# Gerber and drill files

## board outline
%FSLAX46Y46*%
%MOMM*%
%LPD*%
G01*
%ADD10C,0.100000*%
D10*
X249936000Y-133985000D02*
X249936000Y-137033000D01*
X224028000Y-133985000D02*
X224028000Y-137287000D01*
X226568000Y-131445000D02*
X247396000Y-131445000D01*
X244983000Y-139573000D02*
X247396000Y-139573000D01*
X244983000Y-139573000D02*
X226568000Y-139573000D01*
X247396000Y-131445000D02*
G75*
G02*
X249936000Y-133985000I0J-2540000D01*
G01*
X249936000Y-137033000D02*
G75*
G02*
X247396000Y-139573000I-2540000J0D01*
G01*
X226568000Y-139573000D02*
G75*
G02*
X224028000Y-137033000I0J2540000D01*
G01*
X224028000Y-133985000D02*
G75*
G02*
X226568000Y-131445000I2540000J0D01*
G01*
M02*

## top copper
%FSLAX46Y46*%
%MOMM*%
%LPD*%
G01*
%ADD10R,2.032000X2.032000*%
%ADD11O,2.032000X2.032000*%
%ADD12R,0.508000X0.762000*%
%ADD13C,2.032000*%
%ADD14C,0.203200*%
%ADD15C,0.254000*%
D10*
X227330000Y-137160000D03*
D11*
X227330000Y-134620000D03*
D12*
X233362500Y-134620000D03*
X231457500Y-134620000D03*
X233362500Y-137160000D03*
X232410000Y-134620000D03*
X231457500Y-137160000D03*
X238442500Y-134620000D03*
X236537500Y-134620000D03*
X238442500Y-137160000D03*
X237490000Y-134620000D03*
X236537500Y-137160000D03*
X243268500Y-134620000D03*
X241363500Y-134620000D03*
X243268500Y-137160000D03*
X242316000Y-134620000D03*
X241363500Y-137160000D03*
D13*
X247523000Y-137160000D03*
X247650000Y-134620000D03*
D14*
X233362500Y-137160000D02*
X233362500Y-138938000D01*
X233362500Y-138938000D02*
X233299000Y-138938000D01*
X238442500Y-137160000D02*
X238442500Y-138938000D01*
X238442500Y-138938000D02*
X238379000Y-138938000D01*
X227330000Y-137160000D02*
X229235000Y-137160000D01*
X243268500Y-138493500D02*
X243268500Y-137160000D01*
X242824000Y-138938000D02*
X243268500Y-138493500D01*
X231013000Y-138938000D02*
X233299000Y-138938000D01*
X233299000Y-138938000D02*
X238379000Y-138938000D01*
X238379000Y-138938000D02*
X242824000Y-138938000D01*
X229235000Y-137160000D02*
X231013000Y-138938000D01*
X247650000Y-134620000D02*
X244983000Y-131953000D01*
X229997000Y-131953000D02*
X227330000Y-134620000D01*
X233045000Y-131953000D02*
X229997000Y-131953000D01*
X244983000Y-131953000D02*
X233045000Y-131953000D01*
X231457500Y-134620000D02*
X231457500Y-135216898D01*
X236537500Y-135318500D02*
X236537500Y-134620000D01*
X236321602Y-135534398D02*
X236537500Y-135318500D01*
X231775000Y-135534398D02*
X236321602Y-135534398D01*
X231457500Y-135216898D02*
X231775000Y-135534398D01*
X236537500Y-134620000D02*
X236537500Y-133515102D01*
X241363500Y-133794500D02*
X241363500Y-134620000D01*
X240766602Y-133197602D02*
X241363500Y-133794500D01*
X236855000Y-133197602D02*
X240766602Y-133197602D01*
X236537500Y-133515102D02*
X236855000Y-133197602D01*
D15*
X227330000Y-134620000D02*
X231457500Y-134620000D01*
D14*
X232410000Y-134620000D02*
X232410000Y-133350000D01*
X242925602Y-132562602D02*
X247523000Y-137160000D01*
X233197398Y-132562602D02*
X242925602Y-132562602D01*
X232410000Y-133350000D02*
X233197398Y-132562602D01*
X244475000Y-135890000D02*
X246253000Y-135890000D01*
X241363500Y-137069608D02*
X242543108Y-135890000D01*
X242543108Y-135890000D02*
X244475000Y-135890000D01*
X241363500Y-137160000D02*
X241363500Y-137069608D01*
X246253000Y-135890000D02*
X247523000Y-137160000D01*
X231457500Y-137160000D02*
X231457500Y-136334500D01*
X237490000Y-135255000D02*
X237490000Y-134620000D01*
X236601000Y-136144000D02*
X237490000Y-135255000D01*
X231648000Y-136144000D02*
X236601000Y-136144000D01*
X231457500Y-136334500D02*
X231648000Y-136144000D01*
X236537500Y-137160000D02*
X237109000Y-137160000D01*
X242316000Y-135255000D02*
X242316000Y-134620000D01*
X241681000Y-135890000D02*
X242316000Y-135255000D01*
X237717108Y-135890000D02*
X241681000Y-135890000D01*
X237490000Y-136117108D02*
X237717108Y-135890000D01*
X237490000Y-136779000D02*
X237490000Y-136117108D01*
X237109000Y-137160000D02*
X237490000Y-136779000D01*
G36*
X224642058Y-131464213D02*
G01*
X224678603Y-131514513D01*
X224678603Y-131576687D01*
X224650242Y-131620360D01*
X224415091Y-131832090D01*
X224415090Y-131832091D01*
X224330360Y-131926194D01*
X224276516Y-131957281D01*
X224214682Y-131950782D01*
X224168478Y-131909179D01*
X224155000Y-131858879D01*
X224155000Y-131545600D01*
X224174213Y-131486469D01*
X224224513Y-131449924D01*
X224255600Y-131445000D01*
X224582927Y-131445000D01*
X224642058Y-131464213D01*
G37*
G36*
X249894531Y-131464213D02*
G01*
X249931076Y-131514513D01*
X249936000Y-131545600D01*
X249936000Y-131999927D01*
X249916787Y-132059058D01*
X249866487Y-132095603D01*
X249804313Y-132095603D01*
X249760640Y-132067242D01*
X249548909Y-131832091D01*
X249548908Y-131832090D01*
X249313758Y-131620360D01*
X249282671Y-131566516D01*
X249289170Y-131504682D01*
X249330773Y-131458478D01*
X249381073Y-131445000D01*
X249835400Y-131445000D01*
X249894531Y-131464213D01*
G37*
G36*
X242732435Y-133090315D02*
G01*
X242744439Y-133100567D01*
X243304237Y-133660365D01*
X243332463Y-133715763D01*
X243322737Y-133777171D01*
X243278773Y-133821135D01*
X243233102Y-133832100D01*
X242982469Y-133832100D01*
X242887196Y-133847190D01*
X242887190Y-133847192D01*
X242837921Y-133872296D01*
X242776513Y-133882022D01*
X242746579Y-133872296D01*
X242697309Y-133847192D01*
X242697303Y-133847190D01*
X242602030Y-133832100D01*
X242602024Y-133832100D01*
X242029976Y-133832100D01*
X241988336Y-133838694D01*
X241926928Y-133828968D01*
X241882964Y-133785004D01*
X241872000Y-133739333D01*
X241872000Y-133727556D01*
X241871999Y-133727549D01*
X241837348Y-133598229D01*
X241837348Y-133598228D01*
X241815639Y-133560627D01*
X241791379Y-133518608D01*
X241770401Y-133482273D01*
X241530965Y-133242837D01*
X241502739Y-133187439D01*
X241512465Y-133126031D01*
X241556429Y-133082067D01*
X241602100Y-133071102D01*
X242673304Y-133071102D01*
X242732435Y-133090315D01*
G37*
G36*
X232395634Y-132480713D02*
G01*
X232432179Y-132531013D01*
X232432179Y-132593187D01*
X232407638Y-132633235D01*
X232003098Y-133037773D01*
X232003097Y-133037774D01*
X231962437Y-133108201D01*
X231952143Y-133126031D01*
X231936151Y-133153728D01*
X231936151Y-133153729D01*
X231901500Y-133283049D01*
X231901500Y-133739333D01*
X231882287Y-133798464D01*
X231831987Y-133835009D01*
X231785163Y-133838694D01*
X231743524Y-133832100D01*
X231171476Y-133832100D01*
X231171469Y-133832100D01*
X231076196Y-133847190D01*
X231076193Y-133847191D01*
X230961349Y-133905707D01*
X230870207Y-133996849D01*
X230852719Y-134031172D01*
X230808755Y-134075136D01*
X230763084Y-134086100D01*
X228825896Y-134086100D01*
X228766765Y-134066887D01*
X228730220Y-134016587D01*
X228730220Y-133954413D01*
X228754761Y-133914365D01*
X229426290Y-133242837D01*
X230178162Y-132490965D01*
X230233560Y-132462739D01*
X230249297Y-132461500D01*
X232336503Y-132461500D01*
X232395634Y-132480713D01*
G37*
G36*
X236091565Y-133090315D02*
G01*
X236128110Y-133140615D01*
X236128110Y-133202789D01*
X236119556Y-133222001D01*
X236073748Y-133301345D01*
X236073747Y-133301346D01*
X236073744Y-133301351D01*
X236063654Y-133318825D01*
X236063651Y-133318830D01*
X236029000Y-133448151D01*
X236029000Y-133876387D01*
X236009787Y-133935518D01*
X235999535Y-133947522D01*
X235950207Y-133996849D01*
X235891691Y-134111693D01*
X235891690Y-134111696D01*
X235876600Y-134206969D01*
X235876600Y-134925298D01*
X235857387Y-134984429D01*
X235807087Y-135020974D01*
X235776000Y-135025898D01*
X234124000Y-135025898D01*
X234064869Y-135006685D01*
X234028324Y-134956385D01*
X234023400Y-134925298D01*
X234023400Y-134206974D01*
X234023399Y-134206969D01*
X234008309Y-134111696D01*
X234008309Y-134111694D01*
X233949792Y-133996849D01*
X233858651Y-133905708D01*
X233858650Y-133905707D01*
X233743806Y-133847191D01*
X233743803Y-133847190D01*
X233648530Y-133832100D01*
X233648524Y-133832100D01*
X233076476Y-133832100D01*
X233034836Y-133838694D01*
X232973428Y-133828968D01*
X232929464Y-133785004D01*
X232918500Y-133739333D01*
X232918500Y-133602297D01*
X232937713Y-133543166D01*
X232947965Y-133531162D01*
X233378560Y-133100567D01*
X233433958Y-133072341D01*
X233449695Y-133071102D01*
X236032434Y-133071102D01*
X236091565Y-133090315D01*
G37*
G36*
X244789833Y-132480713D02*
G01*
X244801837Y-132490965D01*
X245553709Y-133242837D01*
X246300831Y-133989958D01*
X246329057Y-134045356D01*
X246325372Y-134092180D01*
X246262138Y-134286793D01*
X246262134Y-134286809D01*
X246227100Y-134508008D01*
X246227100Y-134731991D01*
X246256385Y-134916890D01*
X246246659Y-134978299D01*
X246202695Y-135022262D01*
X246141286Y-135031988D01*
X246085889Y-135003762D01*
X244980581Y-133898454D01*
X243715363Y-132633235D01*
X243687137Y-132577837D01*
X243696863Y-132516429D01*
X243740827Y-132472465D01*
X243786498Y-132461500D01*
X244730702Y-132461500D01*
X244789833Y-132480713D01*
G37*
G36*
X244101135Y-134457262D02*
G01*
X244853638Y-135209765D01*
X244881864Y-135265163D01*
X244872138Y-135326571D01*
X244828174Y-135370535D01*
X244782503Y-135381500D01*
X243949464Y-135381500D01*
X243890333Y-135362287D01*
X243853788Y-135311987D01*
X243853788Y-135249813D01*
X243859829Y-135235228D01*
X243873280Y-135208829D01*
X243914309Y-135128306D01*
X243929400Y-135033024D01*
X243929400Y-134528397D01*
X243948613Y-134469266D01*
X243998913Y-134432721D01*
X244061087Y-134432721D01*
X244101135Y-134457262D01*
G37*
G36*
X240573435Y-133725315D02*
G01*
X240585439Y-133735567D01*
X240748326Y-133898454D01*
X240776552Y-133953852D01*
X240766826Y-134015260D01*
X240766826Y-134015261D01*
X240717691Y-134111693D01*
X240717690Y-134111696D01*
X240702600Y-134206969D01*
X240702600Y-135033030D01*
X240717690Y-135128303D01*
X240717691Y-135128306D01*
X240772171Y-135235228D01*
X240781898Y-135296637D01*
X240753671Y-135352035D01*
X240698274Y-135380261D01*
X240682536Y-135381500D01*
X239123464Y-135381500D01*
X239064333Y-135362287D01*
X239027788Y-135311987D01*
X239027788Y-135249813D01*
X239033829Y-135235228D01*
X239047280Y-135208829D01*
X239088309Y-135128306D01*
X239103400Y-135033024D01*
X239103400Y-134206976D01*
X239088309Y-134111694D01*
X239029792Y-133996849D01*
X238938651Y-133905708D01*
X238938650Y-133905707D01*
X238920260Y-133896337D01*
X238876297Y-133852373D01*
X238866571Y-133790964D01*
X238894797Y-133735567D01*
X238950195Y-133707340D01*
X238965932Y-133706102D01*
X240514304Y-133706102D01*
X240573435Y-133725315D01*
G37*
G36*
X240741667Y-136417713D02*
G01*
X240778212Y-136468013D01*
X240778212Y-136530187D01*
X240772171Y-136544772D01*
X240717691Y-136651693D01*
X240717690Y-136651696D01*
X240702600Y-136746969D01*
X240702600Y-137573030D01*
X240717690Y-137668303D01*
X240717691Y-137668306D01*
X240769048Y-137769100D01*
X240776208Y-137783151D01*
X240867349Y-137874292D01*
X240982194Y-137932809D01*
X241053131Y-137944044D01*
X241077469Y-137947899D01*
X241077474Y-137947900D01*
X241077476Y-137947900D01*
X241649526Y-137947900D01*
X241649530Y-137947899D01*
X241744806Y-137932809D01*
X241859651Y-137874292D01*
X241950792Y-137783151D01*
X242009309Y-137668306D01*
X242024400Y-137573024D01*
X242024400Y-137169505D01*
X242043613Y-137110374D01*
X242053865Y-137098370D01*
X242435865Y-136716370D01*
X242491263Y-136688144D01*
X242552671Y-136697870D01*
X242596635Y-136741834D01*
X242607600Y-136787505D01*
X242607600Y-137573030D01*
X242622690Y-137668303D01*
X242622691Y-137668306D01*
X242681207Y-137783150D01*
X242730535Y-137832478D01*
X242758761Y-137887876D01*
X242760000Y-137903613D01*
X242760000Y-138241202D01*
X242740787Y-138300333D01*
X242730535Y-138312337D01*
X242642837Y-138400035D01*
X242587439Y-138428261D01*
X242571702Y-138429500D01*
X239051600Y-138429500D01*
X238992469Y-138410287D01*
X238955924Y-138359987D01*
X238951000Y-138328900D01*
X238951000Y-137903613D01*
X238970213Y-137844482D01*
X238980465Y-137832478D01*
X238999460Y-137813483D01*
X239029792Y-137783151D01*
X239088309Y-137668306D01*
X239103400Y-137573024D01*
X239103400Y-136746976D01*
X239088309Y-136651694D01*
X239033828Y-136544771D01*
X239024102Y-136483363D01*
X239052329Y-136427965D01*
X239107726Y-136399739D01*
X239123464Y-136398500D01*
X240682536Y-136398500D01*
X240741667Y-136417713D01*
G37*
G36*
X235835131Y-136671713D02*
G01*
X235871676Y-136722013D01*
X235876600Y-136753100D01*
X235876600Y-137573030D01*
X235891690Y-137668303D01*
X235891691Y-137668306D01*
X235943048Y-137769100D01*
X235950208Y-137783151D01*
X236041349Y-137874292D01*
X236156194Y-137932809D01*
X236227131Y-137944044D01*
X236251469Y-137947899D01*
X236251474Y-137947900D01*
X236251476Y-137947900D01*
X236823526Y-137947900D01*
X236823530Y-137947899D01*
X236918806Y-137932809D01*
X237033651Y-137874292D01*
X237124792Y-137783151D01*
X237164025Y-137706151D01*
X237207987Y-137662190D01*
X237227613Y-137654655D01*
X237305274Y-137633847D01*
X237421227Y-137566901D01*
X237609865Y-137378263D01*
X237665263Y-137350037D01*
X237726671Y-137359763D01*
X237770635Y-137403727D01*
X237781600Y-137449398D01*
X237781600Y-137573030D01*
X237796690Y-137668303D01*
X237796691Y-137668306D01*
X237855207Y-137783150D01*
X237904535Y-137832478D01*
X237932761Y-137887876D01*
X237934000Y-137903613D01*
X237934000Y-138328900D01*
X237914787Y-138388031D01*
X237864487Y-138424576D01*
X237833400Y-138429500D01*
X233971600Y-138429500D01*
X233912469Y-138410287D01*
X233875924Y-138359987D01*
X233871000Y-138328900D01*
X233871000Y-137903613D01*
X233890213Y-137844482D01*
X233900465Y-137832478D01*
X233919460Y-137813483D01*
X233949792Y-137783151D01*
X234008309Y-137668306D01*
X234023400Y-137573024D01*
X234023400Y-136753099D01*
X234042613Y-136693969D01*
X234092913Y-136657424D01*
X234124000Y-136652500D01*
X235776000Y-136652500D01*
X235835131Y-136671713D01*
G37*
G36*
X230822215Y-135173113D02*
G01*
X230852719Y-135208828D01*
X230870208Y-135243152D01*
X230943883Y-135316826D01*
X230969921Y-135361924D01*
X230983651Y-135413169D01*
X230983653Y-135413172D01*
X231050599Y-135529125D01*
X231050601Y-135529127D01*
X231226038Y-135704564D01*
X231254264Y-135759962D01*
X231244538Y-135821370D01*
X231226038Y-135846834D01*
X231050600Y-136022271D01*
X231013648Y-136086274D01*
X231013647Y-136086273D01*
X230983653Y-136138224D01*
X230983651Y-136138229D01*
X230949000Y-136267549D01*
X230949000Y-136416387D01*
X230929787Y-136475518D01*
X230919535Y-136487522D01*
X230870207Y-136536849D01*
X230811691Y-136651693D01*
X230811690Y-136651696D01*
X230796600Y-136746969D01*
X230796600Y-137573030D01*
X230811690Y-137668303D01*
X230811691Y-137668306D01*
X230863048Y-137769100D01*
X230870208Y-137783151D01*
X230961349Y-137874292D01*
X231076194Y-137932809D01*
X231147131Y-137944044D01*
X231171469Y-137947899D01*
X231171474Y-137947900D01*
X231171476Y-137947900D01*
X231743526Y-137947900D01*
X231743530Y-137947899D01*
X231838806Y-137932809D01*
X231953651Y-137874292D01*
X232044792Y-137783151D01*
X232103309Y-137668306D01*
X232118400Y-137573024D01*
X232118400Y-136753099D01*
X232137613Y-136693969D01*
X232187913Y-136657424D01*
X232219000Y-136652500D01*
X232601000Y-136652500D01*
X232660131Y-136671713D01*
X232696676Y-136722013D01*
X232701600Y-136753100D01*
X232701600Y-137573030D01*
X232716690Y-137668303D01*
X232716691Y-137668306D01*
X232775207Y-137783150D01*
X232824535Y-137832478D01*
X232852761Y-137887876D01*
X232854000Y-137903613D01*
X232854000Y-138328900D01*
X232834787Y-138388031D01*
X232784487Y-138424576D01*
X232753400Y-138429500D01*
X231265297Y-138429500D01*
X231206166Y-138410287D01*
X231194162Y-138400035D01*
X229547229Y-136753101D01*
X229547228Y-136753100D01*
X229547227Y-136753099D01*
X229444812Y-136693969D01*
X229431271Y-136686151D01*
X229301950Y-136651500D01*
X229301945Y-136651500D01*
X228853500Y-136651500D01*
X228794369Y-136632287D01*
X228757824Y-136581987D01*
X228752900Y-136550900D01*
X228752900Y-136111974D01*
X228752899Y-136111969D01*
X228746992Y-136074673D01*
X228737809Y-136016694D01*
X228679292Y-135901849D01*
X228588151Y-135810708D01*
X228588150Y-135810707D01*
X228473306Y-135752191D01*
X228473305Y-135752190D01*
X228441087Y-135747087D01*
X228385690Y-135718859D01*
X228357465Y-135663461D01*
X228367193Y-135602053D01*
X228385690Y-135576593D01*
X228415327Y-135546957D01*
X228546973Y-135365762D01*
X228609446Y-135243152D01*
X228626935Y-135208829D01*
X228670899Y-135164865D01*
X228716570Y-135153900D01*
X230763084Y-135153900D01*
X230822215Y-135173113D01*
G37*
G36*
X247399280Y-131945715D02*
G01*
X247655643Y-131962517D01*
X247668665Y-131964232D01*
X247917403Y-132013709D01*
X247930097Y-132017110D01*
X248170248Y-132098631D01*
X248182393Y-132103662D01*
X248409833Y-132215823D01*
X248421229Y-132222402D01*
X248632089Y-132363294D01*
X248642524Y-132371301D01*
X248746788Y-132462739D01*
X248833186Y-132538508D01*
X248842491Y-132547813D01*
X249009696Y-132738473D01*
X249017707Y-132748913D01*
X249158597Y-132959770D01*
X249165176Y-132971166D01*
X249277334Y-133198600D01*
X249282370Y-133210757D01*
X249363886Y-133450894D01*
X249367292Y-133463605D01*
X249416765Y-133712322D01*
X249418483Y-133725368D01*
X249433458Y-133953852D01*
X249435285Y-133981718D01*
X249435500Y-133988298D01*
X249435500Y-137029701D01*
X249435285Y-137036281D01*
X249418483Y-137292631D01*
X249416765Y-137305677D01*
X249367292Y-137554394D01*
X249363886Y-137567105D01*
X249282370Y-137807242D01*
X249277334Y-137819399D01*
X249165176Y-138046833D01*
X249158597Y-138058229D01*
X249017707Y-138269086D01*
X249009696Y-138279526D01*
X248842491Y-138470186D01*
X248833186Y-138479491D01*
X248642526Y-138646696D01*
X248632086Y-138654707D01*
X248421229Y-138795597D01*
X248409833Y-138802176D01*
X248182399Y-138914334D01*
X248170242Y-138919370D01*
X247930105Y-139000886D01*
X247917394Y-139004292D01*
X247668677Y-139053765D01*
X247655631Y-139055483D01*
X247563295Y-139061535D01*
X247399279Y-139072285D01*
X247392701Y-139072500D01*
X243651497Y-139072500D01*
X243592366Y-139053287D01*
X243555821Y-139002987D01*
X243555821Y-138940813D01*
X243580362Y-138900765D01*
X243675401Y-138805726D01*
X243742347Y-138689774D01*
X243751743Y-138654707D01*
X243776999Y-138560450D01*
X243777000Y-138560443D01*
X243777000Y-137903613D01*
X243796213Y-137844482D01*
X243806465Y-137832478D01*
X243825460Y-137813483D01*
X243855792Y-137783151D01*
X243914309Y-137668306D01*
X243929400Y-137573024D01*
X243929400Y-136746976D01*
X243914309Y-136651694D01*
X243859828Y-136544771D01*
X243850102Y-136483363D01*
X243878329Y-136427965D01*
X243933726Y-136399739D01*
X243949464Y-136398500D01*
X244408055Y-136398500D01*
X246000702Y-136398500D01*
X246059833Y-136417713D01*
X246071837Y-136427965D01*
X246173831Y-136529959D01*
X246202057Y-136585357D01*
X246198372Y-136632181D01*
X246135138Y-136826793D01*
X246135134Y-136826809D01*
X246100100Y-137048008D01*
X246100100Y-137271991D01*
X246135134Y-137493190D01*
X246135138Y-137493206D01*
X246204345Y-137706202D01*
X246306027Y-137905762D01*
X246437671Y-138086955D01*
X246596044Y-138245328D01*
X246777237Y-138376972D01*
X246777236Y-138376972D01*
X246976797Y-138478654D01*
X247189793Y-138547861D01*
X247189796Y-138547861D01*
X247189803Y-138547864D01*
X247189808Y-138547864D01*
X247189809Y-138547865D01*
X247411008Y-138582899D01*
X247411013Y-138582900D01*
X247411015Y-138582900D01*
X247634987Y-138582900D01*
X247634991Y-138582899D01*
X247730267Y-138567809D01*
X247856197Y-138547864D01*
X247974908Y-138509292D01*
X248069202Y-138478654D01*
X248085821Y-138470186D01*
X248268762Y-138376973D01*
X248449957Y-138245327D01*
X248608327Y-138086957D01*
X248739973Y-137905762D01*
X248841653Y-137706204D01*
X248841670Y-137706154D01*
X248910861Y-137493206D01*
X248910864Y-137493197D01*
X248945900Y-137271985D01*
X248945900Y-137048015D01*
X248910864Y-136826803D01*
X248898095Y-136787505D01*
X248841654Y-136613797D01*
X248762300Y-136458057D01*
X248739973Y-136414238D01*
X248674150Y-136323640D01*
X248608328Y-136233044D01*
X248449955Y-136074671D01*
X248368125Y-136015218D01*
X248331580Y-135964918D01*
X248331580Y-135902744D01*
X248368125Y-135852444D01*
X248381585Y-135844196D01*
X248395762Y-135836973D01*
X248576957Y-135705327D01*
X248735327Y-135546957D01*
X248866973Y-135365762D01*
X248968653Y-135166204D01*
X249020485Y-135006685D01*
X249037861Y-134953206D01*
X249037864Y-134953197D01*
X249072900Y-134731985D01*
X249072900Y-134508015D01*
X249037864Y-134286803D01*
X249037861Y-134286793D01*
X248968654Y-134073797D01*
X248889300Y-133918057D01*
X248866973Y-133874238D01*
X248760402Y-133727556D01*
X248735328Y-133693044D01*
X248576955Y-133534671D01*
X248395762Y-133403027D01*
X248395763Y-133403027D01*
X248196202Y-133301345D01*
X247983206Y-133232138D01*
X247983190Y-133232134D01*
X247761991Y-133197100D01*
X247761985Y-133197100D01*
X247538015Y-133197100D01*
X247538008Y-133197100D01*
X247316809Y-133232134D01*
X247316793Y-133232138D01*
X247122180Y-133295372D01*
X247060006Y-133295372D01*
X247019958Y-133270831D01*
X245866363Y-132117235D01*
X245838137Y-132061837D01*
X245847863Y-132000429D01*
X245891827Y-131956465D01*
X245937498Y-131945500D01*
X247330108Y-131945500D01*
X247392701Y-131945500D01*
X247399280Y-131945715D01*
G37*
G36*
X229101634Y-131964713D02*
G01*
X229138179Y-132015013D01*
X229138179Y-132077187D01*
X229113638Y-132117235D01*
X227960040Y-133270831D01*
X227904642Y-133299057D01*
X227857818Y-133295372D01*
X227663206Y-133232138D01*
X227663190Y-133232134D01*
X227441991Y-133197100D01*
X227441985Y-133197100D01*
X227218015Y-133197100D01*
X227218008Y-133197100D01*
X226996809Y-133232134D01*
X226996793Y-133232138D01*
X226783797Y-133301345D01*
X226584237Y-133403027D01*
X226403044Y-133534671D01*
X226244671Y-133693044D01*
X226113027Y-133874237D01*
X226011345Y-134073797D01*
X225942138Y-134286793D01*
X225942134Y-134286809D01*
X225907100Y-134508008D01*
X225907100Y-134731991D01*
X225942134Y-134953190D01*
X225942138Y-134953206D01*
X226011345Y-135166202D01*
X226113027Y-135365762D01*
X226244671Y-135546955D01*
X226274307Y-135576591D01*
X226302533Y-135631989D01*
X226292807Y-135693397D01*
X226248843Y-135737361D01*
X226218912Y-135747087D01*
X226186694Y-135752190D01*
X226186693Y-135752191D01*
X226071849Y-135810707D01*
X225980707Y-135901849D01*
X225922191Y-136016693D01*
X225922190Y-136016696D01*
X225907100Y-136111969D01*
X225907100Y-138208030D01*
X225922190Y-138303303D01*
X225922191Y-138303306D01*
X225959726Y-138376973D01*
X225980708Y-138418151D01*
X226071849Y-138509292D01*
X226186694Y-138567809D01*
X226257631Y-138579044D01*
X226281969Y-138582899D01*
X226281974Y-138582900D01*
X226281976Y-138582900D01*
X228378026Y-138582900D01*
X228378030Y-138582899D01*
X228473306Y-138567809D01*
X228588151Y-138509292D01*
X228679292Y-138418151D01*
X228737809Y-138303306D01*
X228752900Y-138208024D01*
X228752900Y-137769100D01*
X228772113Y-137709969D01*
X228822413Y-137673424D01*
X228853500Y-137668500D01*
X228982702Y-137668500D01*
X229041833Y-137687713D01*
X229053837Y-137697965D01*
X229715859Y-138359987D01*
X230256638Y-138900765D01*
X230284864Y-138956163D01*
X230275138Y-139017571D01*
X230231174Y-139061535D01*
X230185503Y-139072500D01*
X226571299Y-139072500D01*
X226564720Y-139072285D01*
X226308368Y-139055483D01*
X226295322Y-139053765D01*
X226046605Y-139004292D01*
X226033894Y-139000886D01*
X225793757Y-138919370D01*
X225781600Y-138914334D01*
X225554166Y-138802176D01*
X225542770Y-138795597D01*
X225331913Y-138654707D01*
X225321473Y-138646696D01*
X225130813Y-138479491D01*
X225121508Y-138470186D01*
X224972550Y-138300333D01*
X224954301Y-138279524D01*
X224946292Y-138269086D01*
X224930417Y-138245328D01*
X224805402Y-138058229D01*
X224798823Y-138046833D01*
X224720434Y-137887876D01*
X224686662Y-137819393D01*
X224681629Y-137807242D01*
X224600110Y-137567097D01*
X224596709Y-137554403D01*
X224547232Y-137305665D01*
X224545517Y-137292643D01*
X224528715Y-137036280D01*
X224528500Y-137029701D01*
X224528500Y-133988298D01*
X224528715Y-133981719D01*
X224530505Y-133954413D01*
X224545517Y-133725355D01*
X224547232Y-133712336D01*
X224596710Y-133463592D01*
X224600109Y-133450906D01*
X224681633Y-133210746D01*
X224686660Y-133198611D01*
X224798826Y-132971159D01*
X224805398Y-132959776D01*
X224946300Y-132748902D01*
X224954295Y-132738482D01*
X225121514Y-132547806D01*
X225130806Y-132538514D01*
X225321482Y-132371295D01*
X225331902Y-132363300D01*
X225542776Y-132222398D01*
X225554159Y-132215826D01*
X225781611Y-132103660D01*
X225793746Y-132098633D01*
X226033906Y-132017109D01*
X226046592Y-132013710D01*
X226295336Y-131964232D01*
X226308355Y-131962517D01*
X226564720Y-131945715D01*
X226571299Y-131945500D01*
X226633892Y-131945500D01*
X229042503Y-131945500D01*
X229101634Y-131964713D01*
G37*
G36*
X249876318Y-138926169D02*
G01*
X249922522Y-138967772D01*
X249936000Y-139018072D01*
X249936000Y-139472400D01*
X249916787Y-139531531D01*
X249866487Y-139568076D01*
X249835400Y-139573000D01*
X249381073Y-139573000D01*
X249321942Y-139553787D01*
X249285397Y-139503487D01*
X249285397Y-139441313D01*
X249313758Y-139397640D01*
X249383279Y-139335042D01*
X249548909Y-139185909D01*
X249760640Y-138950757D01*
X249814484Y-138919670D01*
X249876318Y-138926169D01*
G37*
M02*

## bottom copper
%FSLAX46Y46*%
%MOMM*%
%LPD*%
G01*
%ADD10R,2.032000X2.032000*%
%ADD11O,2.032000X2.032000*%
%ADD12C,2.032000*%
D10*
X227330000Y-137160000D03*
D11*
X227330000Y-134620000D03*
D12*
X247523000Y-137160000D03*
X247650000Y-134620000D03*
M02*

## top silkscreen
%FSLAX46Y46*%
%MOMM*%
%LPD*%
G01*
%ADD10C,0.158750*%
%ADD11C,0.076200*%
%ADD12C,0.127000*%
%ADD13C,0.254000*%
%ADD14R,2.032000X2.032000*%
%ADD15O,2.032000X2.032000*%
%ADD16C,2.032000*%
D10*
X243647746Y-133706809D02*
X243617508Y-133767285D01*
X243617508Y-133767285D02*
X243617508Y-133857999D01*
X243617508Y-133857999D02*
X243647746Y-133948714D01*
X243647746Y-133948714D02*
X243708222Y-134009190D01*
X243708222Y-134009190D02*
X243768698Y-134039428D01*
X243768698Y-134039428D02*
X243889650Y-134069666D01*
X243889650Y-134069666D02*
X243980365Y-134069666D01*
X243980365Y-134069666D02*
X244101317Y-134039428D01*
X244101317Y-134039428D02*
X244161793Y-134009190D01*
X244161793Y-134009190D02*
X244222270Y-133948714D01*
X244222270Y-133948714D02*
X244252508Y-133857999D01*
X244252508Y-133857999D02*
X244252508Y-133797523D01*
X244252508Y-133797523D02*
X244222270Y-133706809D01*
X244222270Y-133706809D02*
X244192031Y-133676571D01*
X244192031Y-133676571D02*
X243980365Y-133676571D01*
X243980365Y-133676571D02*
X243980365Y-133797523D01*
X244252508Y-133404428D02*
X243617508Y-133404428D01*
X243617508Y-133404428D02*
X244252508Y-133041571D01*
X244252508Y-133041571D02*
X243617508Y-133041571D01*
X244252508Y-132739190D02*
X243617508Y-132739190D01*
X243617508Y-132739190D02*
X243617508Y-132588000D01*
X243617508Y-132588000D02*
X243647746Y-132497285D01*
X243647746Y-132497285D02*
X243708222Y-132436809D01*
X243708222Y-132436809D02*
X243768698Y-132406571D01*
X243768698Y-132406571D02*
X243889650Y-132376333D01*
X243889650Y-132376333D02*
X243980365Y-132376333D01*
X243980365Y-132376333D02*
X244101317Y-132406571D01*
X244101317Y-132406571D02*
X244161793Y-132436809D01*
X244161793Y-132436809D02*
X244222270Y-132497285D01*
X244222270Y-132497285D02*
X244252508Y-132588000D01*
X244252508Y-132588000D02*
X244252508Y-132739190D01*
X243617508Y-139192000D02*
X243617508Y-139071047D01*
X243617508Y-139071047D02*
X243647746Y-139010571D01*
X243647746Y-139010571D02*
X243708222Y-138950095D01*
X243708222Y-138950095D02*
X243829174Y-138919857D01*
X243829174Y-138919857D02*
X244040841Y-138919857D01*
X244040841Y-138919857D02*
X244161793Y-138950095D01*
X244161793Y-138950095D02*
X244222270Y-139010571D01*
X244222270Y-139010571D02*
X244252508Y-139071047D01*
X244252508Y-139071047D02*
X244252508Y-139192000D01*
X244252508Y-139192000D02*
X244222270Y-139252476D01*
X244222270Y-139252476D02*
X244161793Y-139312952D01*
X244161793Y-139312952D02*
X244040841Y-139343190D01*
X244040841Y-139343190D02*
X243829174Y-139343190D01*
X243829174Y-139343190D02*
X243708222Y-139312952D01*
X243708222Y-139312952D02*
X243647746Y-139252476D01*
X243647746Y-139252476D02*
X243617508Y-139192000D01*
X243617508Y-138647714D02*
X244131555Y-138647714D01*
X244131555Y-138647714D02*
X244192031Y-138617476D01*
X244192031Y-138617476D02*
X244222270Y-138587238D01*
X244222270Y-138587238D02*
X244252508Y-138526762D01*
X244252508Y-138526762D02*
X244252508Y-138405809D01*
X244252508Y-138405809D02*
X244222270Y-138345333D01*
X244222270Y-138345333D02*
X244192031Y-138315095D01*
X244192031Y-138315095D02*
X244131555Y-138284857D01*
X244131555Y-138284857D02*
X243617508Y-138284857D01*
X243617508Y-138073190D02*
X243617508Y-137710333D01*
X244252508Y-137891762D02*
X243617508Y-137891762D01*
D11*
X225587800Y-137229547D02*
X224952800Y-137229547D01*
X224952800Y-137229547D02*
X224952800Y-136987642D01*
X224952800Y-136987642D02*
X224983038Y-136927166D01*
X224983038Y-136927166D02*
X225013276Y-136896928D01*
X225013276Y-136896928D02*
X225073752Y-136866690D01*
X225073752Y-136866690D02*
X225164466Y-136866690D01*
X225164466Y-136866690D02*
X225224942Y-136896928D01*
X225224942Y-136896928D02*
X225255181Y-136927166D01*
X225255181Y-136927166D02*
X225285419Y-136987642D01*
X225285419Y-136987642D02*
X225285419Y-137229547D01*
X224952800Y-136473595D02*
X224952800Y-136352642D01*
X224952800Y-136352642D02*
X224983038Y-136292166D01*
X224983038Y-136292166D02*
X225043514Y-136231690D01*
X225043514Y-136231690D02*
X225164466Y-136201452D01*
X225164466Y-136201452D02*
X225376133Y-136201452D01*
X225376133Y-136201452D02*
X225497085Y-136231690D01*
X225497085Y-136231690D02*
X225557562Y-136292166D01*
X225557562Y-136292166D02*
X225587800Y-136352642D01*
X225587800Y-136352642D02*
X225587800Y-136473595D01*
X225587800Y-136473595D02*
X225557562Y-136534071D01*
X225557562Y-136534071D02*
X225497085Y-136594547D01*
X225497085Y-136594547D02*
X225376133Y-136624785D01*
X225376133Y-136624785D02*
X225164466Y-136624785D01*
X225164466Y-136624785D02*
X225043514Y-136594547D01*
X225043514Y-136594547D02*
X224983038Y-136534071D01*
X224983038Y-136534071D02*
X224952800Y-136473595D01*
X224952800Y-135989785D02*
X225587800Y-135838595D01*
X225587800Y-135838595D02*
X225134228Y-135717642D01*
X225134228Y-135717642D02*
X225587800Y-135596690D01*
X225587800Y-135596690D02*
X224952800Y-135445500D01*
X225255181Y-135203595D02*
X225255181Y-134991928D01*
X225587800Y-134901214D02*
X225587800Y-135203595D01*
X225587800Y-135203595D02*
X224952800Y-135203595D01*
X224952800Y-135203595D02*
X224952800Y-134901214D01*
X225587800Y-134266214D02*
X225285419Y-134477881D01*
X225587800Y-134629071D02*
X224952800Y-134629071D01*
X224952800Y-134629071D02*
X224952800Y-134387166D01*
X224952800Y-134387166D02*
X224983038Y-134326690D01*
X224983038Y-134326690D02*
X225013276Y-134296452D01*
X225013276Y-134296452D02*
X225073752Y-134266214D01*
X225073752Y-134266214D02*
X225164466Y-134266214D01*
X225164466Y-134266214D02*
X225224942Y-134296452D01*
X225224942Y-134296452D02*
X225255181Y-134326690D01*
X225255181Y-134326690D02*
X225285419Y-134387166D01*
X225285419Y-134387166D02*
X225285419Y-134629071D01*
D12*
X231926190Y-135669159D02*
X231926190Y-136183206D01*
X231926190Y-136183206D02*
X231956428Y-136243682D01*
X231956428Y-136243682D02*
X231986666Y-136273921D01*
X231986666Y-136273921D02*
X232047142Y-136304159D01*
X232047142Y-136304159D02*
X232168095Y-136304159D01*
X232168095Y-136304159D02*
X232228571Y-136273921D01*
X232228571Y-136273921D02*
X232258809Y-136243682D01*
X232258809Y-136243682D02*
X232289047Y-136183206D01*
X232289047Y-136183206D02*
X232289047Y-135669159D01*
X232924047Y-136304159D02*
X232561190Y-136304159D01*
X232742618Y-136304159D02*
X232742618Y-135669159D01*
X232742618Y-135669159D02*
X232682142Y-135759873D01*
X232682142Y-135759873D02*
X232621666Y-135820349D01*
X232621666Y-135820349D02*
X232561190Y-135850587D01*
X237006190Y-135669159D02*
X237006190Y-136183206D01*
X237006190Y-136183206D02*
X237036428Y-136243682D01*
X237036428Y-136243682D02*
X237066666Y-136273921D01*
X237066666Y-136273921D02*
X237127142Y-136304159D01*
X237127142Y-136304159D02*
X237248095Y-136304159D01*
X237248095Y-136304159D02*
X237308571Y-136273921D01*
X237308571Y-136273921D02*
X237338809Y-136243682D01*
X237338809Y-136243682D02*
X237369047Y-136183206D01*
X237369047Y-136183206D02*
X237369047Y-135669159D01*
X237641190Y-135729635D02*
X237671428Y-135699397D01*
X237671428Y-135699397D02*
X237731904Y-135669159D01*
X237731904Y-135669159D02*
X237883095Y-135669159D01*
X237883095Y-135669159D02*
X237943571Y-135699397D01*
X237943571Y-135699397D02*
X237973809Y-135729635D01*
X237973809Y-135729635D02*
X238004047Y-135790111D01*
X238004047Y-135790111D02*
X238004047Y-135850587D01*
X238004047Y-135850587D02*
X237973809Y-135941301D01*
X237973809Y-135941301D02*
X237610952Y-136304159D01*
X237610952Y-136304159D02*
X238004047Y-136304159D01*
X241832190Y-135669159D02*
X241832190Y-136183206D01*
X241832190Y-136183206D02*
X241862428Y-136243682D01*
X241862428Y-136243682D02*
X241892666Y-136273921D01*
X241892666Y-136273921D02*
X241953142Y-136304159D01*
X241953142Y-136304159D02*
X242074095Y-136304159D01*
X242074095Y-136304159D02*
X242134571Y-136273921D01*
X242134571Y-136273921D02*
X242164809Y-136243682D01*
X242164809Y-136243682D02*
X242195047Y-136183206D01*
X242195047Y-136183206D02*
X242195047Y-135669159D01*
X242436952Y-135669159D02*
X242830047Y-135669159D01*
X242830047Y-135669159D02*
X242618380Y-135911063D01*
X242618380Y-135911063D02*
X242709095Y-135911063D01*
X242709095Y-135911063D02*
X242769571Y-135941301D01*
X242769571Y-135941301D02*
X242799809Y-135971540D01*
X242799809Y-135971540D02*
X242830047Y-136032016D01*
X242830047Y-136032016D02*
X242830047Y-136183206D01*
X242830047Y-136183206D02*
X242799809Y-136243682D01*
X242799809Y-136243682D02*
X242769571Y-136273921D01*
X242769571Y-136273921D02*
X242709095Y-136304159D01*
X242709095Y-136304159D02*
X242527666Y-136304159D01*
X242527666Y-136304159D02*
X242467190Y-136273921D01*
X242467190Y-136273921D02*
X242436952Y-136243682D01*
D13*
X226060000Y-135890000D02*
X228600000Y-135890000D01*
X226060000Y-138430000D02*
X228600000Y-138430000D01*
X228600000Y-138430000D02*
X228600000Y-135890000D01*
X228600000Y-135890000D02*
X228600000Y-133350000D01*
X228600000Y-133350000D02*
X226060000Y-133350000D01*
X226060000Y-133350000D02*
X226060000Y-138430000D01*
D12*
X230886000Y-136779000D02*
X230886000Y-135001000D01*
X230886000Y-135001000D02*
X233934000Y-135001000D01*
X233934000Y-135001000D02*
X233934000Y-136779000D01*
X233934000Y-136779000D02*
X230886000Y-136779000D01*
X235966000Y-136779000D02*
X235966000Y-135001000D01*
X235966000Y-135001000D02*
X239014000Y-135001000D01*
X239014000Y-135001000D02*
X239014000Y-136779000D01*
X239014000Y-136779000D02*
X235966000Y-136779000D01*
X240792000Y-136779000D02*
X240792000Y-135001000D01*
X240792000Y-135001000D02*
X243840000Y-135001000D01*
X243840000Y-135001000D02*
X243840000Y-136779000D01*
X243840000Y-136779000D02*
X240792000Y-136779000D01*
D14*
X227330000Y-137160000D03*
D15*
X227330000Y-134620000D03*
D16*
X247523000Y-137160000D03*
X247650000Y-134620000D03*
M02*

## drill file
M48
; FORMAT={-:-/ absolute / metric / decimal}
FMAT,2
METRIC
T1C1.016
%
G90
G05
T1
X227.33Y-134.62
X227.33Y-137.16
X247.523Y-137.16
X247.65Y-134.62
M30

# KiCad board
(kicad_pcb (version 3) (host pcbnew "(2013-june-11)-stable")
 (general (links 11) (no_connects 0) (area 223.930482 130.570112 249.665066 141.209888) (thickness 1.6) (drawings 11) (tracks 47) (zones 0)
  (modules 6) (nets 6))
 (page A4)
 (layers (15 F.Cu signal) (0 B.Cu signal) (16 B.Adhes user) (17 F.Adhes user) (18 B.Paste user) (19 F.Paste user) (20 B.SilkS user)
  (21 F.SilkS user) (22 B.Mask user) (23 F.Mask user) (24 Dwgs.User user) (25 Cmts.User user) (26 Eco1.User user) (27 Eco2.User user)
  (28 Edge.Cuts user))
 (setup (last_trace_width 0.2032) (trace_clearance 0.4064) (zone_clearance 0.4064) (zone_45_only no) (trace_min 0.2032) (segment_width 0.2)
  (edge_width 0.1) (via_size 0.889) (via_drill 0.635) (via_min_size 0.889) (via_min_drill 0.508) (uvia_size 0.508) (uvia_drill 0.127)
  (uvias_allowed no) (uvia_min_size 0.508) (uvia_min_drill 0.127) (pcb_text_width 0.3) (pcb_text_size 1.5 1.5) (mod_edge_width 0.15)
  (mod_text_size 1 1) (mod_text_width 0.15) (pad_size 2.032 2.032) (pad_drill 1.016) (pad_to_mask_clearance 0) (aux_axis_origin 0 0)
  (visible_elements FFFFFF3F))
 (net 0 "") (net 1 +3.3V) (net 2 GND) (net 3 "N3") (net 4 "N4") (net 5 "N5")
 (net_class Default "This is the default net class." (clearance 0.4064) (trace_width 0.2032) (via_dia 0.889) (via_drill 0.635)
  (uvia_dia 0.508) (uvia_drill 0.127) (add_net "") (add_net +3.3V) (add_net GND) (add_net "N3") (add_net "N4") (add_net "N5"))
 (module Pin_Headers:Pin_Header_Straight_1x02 (layer F.Cu) (at 227.33 135.89 90)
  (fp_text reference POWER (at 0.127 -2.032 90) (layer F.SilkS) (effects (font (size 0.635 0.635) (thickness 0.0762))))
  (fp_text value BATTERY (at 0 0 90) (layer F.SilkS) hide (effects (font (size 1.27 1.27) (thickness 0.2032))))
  (fp_line (start 0 -1.27) (end 0 1.27) (layer F.SilkS) (width 0.254))
  (fp_line (start -2.54 -1.27) (end -2.54 1.27) (layer F.SilkS) (width 0.254))
  (fp_line (start -2.54 1.27) (end 0 1.27) (layer F.SilkS) (width 0.254))
  (fp_line (start 0 1.27) (end 2.54 1.27) (layer F.SilkS) (width 0.254))
  (fp_line (start 2.54 1.27) (end 2.54 -1.27) (layer F.SilkS) (width 0.254))
  (fp_line (start 2.54 -1.27) (end -2.54 -1.27) (layer F.SilkS) (width 0.254))
  (pad 1 thru_hole rect (at -1.27 0 90) (size 2.032 2.032) (drill 1.016) (layers *.Cu *.Mask F.SilkS) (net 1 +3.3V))
  (pad 2 thru_hole oval (at 1.27 0 90) (size 2.032 2.032) (drill 1.016) (layers *.Cu *.Mask F.SilkS) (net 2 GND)))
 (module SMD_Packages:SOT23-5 (layer F.Cu) (at 232.41 135.89 180)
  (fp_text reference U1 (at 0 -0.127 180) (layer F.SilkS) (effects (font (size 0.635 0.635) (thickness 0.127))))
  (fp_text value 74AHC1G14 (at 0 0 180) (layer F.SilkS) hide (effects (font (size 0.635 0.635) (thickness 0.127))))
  (fp_line (start 1.524 -0.889) (end 1.524 0.889) (layer F.SilkS) (width 0.127))
  (fp_line (start 1.524 0.889) (end -1.524 0.889) (layer F.SilkS) (width 0.127))
  (fp_line (start -1.524 0.889) (end -1.524 -0.889) (layer F.SilkS) (width 0.127))
  (fp_line (start -1.524 -0.889) (end 1.524 -0.889) (layer F.SilkS) (width 0.127))
  (pad 1 smd rect (at -0.9525 1.27 180) (size 0.508 0.762) (layers F.Cu F.Paste F.Mask))
  (pad 3 smd rect (at 0.9525 1.27 180) (size 0.508 0.762) (layers F.Cu F.Paste F.Mask) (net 2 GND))
  (pad 5 smd rect (at -0.9525 -1.27 180) (size 0.508 0.762) (layers F.Cu F.Paste F.Mask) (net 1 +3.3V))
  (pad 2 smd rect (at 0 1.27 180) (size 0.508 0.762) (layers F.Cu F.Paste F.Mask) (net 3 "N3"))
  (pad 4 smd rect (at 0.9525 -1.27 180) (size 0.508 0.762) (layers F.Cu F.Paste F.Mask) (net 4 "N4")))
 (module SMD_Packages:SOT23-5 (layer F.Cu) (at 237.49 135.89 180)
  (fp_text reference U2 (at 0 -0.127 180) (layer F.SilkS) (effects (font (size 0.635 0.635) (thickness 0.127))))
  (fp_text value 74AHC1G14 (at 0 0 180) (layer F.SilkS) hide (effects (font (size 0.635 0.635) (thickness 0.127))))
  (fp_line (start 1.524 -0.889) (end 1.524 0.889) (layer F.SilkS) (width 0.127))
  (fp_line (start 1.524 0.889) (end -1.524 0.889) (layer F.SilkS) (width 0.127))
  (fp_line (start -1.524 0.889) (end -1.524 -0.889) (layer F.SilkS) (width 0.127))
  (fp_line (start -1.524 -0.889) (end 1.524 -0.889) (layer F.SilkS) (width 0.127))
  (pad 1 smd rect (at -0.9525 1.27 180) (size 0.508 0.762) (layers F.Cu F.Paste F.Mask))
  (pad 3 smd rect (at 0.9525 1.27 180) (size 0.508 0.762) (layers F.Cu F.Paste F.Mask) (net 2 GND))
  (pad 5 smd rect (at -0.9525 -1.27 180) (size 0.508 0.762) (layers F.Cu F.Paste F.Mask) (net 1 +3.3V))
  (pad 2 smd rect (at 0 1.27 180) (size 0.508 0.762) (layers F.Cu F.Paste F.Mask) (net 4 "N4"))
  (pad 4 smd rect (at 0.9525 -1.27 180) (size 0.508 0.762) (layers F.Cu F.Paste F.Mask) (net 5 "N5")))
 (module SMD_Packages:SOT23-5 (layer F.Cu) (at 242.316 135.89 180)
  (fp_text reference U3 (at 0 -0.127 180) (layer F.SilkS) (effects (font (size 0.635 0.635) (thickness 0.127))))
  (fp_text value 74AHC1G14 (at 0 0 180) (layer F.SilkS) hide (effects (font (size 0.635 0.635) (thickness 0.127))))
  (fp_line (start 1.524 -0.889) (end 1.524 0.889) (layer F.SilkS) (width 0.127))
  (fp_line (start 1.524 0.889) (end -1.524 0.889) (layer F.SilkS) (width 0.127))
  (fp_line (start -1.524 0.889) (end -1.524 -0.889) (layer F.SilkS) (width 0.127))
  (fp_line (start -1.524 -0.889) (end 1.524 -0.889) (layer F.SilkS) (width 0.127))
  (pad 1 smd rect (at -0.9525 1.27 180) (size 0.508 0.762) (layers F.Cu F.Paste F.Mask))
  (pad 3 smd rect (at 0.9525 1.27 180) (size 0.508 0.762) (layers F.Cu F.Paste F.Mask) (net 2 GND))
  (pad 5 smd rect (at -0.9525 -1.27 180) (size 0.508 0.762) (layers F.Cu F.Paste F.Mask) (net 1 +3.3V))
  (pad 2 smd rect (at 0 1.27 180) (size 0.508 0.762) (layers F.Cu F.Paste F.Mask) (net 5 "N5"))
  (pad 4 smd rect (at 0.9525 -1.27 180) (size 0.508 0.762) (layers F.Cu F.Paste F.Mask) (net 3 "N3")))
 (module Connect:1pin (layer F.Cu) (at 247.523 137.16)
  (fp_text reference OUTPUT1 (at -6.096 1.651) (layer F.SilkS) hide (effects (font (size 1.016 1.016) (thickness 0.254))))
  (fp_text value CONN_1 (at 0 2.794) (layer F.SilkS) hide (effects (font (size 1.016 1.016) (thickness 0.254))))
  (pad 1 thru_hole circle (at 0 0) (size 2.032 2.032) (drill 1.016) (layers *.Cu *.Mask F.SilkS) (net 3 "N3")))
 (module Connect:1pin (layer F.Cu) (at 247.65 134.62)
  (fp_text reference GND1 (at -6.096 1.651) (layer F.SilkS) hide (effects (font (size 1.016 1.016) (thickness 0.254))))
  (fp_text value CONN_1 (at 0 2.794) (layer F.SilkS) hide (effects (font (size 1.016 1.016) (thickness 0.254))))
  (pad 1 thru_hole circle (at 0 0) (size 2.032 2.032) (drill 1.016) (layers *.Cu *.Mask F.SilkS) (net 2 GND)))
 (gr_line (start 249.936 133.985) (end 249.936 137.033) (angle 90) (layer Edge.Cuts) (width 0.1))
 (gr_line (start 224.028 133.985) (end 224.028 137.287) (angle 90) (layer Edge.Cuts) (width 0.1))
 (gr_line (start 226.568 131.445) (end 247.396 131.445) (angle 90) (layer Edge.Cuts) (width 0.1))
 (gr_line (start 244.983 139.573) (end 247.396 139.573) (angle 90) (layer Edge.Cuts) (width 0.1))
 (gr_line (start 244.983 139.573) (end 226.568 139.573) (angle 90) (layer Edge.Cuts) (width 0.1))
 (gr_arc (start 247.396 133.985) (end 247.396 131.445) (angle 90) (layer Edge.Cuts) (width 0.1))
 (gr_arc (start 247.396 137.033) (end 249.936 137.033) (angle 90) (layer Edge.Cuts) (width 0.1))
 (gr_arc (start 226.568 137.033) (end 226.568 139.573) (angle 90) (layer Edge.Cuts) (width 0.1))
 (gr_arc (start 226.568 133.985) (end 224.028 133.985) (angle 90) (layer Edge.Cuts) (width 0.1))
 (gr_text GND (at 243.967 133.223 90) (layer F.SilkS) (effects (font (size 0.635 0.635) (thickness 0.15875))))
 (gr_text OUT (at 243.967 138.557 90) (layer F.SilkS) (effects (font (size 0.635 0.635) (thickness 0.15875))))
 (segment (start 233.3625 137.16) (end 233.3625 138.938) (width 0.2032) (layer F.Cu) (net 1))
 (segment (start 233.3625 138.938) (end 233.299 138.938) (width 0.2032) (layer F.Cu) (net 1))
 (segment (start 238.4425 137.16) (end 238.4425 138.938) (width 0.2032) (layer F.Cu) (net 1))
 (segment (start 238.4425 138.938) (end 238.379 138.938) (width 0.2032) (layer F.Cu) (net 1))
 (segment (start 227.33 137.16) (end 229.235 137.16) (width 0.2032) (layer F.Cu) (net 1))
 (segment (start 243.2685 138.4935) (end 243.2685 137.16) (width 0.2032) (layer F.Cu) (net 1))
 (segment (start 242.824 138.938) (end 243.2685 138.4935) (width 0.2032) (layer F.Cu) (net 1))
 (segment (start 231.013 138.938) (end 233.299 138.938) (width 0.2032) (layer F.Cu) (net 1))
 (segment (start 233.299 138.938) (end 238.379 138.938) (width 0.2032) (layer F.Cu) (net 1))
 (segment (start 238.379 138.938) (end 242.824 138.938) (width 0.2032) (layer F.Cu) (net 1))
 (segment (start 229.235 137.16) (end 231.013 138.938) (width 0.2032) (layer F.Cu) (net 1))
 (segment (start 247.65 134.62) (end 244.983 131.953) (width 0.2032) (layer F.Cu) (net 2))
 (segment (start 229.997 131.953) (end 227.33 134.62) (width 0.2032) (layer F.Cu) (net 2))
 (segment (start 233.045 131.953) (end 229.997 131.953) (width 0.2032) (layer F.Cu) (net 2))
 (segment (start 244.983 131.953) (end 233.045 131.953) (width 0.2032) (layer F.Cu) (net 2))
 (segment (start 231.4575 134.62) (end 231.4575 135.216898) (width 0.2032) (layer F.Cu) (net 2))
 (segment (start 236.5375 135.3185) (end 236.5375 134.62) (width 0.2032) (layer F.Cu) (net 2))
 (segment (start 236.321602 135.534398) (end 236.5375 135.3185) (width 0.2032) (layer F.Cu) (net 2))
 (segment (start 231.775 135.534398) (end 236.321602 135.534398) (width 0.2032) (layer F.Cu) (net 2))
 (segment (start 231.4575 135.216898) (end 231.775 135.534398) (width 0.2032) (layer F.Cu) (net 2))
 (segment (start 236.5375 134.62) (end 236.5375 133.515102) (width 0.2032) (layer F.Cu) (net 2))
 (segment (start 241.3635 133.7945) (end 241.3635 134.62) (width 0.2032) (layer F.Cu) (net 2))
 (segment (start 240.766602 133.197602) (end 241.3635 133.7945) (width 0.2032) (layer F.Cu) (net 2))
 (segment (start 236.855 133.197602) (end 240.766602 133.197602) (width 0.2032) (layer F.Cu) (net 2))
 (segment (start 236.5375 133.515102) (end 236.855 133.197602) (width 0.2032) (layer F.Cu) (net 2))
 (segment (start 227.33 134.62) (end 231.4575 134.62) (width 0.254) (layer F.Cu) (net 2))
 (segment (start 232.41 134.62) (end 232.41 133.35) (width 0.2032) (layer F.Cu) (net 3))
 (segment (start 242.925602 132.562602) (end 247.523 137.16) (width 0.2032) (layer F.Cu) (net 3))
 (segment (start 233.197398 132.562602) (end 242.925602 132.562602) (width 0.2032) (layer F.Cu) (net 3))
 (segment (start 232.41 133.35) (end 233.197398 132.562602) (width 0.2032) (layer F.Cu) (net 3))
 (segment (start 244.475 135.89) (end 246.253 135.89) (width 0.2032) (layer F.Cu) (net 3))
 (segment (start 241.3635 137.069608) (end 242.543108 135.89) (width 0.2032) (layer F.Cu) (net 3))
 (segment (start 242.543108 135.89) (end 244.475 135.89) (width 0.2032) (layer F.Cu) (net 3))
 (segment (start 241.3635 137.16) (end 241.3635 137.069608) (width 0.2032) (layer F.Cu) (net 3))
 (segment (start 246.253 135.89) (end 247.523 137.16) (width 0.2032) (layer F.Cu) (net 3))
 (segment (start 231.4575 137.16) (end 231.4575 136.3345) (width 0.2032) (layer F.Cu) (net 4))
 (segment (start 237.49 135.255) (end 237.49 134.62) (width 0.2032) (layer F.Cu) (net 4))
 (segment (start 236.601 136.144) (end 237.49 135.255) (width 0.2032) (layer F.Cu) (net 4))
 (segment (start 231.648 136.144) (end 236.601 136.144) (width 0.2032) (layer F.Cu) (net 4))
 (segment (start 231.4575 136.3345) (end 231.648 136.144) (width 0.2032) (layer F.Cu) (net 4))
 (segment (start 236.5375 137.16) (end 237.109 137.16) (width 0.2032) (layer F.Cu) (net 5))
 (segment (start 242.316 135.255) (end 242.316 134.62) (width 0.2032) (layer F.Cu) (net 5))
 (segment (start 241.681 135.89) (end 242.316 135.255) (width 0.2032) (layer F.Cu) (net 5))
 (segment (start 237.717108 135.89) (end 241.681 135.89) (width 0.2032) (layer F.Cu) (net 5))
 (segment (start 237.49 136.117108) (end 237.717108 135.89) (width 0.2032) (layer F.Cu) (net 5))
 (segment (start 237.49 136.779) (end 237.49 136.117108) (width 0.2032) (layer F.Cu) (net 5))
 (segment (start 237.109 137.16) (end 237.49 136.779) (width 0.2032) (layer F.Cu) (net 5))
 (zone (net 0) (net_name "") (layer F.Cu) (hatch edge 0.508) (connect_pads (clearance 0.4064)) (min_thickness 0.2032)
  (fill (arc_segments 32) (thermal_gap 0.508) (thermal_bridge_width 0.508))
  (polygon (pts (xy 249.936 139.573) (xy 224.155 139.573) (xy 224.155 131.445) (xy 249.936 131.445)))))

